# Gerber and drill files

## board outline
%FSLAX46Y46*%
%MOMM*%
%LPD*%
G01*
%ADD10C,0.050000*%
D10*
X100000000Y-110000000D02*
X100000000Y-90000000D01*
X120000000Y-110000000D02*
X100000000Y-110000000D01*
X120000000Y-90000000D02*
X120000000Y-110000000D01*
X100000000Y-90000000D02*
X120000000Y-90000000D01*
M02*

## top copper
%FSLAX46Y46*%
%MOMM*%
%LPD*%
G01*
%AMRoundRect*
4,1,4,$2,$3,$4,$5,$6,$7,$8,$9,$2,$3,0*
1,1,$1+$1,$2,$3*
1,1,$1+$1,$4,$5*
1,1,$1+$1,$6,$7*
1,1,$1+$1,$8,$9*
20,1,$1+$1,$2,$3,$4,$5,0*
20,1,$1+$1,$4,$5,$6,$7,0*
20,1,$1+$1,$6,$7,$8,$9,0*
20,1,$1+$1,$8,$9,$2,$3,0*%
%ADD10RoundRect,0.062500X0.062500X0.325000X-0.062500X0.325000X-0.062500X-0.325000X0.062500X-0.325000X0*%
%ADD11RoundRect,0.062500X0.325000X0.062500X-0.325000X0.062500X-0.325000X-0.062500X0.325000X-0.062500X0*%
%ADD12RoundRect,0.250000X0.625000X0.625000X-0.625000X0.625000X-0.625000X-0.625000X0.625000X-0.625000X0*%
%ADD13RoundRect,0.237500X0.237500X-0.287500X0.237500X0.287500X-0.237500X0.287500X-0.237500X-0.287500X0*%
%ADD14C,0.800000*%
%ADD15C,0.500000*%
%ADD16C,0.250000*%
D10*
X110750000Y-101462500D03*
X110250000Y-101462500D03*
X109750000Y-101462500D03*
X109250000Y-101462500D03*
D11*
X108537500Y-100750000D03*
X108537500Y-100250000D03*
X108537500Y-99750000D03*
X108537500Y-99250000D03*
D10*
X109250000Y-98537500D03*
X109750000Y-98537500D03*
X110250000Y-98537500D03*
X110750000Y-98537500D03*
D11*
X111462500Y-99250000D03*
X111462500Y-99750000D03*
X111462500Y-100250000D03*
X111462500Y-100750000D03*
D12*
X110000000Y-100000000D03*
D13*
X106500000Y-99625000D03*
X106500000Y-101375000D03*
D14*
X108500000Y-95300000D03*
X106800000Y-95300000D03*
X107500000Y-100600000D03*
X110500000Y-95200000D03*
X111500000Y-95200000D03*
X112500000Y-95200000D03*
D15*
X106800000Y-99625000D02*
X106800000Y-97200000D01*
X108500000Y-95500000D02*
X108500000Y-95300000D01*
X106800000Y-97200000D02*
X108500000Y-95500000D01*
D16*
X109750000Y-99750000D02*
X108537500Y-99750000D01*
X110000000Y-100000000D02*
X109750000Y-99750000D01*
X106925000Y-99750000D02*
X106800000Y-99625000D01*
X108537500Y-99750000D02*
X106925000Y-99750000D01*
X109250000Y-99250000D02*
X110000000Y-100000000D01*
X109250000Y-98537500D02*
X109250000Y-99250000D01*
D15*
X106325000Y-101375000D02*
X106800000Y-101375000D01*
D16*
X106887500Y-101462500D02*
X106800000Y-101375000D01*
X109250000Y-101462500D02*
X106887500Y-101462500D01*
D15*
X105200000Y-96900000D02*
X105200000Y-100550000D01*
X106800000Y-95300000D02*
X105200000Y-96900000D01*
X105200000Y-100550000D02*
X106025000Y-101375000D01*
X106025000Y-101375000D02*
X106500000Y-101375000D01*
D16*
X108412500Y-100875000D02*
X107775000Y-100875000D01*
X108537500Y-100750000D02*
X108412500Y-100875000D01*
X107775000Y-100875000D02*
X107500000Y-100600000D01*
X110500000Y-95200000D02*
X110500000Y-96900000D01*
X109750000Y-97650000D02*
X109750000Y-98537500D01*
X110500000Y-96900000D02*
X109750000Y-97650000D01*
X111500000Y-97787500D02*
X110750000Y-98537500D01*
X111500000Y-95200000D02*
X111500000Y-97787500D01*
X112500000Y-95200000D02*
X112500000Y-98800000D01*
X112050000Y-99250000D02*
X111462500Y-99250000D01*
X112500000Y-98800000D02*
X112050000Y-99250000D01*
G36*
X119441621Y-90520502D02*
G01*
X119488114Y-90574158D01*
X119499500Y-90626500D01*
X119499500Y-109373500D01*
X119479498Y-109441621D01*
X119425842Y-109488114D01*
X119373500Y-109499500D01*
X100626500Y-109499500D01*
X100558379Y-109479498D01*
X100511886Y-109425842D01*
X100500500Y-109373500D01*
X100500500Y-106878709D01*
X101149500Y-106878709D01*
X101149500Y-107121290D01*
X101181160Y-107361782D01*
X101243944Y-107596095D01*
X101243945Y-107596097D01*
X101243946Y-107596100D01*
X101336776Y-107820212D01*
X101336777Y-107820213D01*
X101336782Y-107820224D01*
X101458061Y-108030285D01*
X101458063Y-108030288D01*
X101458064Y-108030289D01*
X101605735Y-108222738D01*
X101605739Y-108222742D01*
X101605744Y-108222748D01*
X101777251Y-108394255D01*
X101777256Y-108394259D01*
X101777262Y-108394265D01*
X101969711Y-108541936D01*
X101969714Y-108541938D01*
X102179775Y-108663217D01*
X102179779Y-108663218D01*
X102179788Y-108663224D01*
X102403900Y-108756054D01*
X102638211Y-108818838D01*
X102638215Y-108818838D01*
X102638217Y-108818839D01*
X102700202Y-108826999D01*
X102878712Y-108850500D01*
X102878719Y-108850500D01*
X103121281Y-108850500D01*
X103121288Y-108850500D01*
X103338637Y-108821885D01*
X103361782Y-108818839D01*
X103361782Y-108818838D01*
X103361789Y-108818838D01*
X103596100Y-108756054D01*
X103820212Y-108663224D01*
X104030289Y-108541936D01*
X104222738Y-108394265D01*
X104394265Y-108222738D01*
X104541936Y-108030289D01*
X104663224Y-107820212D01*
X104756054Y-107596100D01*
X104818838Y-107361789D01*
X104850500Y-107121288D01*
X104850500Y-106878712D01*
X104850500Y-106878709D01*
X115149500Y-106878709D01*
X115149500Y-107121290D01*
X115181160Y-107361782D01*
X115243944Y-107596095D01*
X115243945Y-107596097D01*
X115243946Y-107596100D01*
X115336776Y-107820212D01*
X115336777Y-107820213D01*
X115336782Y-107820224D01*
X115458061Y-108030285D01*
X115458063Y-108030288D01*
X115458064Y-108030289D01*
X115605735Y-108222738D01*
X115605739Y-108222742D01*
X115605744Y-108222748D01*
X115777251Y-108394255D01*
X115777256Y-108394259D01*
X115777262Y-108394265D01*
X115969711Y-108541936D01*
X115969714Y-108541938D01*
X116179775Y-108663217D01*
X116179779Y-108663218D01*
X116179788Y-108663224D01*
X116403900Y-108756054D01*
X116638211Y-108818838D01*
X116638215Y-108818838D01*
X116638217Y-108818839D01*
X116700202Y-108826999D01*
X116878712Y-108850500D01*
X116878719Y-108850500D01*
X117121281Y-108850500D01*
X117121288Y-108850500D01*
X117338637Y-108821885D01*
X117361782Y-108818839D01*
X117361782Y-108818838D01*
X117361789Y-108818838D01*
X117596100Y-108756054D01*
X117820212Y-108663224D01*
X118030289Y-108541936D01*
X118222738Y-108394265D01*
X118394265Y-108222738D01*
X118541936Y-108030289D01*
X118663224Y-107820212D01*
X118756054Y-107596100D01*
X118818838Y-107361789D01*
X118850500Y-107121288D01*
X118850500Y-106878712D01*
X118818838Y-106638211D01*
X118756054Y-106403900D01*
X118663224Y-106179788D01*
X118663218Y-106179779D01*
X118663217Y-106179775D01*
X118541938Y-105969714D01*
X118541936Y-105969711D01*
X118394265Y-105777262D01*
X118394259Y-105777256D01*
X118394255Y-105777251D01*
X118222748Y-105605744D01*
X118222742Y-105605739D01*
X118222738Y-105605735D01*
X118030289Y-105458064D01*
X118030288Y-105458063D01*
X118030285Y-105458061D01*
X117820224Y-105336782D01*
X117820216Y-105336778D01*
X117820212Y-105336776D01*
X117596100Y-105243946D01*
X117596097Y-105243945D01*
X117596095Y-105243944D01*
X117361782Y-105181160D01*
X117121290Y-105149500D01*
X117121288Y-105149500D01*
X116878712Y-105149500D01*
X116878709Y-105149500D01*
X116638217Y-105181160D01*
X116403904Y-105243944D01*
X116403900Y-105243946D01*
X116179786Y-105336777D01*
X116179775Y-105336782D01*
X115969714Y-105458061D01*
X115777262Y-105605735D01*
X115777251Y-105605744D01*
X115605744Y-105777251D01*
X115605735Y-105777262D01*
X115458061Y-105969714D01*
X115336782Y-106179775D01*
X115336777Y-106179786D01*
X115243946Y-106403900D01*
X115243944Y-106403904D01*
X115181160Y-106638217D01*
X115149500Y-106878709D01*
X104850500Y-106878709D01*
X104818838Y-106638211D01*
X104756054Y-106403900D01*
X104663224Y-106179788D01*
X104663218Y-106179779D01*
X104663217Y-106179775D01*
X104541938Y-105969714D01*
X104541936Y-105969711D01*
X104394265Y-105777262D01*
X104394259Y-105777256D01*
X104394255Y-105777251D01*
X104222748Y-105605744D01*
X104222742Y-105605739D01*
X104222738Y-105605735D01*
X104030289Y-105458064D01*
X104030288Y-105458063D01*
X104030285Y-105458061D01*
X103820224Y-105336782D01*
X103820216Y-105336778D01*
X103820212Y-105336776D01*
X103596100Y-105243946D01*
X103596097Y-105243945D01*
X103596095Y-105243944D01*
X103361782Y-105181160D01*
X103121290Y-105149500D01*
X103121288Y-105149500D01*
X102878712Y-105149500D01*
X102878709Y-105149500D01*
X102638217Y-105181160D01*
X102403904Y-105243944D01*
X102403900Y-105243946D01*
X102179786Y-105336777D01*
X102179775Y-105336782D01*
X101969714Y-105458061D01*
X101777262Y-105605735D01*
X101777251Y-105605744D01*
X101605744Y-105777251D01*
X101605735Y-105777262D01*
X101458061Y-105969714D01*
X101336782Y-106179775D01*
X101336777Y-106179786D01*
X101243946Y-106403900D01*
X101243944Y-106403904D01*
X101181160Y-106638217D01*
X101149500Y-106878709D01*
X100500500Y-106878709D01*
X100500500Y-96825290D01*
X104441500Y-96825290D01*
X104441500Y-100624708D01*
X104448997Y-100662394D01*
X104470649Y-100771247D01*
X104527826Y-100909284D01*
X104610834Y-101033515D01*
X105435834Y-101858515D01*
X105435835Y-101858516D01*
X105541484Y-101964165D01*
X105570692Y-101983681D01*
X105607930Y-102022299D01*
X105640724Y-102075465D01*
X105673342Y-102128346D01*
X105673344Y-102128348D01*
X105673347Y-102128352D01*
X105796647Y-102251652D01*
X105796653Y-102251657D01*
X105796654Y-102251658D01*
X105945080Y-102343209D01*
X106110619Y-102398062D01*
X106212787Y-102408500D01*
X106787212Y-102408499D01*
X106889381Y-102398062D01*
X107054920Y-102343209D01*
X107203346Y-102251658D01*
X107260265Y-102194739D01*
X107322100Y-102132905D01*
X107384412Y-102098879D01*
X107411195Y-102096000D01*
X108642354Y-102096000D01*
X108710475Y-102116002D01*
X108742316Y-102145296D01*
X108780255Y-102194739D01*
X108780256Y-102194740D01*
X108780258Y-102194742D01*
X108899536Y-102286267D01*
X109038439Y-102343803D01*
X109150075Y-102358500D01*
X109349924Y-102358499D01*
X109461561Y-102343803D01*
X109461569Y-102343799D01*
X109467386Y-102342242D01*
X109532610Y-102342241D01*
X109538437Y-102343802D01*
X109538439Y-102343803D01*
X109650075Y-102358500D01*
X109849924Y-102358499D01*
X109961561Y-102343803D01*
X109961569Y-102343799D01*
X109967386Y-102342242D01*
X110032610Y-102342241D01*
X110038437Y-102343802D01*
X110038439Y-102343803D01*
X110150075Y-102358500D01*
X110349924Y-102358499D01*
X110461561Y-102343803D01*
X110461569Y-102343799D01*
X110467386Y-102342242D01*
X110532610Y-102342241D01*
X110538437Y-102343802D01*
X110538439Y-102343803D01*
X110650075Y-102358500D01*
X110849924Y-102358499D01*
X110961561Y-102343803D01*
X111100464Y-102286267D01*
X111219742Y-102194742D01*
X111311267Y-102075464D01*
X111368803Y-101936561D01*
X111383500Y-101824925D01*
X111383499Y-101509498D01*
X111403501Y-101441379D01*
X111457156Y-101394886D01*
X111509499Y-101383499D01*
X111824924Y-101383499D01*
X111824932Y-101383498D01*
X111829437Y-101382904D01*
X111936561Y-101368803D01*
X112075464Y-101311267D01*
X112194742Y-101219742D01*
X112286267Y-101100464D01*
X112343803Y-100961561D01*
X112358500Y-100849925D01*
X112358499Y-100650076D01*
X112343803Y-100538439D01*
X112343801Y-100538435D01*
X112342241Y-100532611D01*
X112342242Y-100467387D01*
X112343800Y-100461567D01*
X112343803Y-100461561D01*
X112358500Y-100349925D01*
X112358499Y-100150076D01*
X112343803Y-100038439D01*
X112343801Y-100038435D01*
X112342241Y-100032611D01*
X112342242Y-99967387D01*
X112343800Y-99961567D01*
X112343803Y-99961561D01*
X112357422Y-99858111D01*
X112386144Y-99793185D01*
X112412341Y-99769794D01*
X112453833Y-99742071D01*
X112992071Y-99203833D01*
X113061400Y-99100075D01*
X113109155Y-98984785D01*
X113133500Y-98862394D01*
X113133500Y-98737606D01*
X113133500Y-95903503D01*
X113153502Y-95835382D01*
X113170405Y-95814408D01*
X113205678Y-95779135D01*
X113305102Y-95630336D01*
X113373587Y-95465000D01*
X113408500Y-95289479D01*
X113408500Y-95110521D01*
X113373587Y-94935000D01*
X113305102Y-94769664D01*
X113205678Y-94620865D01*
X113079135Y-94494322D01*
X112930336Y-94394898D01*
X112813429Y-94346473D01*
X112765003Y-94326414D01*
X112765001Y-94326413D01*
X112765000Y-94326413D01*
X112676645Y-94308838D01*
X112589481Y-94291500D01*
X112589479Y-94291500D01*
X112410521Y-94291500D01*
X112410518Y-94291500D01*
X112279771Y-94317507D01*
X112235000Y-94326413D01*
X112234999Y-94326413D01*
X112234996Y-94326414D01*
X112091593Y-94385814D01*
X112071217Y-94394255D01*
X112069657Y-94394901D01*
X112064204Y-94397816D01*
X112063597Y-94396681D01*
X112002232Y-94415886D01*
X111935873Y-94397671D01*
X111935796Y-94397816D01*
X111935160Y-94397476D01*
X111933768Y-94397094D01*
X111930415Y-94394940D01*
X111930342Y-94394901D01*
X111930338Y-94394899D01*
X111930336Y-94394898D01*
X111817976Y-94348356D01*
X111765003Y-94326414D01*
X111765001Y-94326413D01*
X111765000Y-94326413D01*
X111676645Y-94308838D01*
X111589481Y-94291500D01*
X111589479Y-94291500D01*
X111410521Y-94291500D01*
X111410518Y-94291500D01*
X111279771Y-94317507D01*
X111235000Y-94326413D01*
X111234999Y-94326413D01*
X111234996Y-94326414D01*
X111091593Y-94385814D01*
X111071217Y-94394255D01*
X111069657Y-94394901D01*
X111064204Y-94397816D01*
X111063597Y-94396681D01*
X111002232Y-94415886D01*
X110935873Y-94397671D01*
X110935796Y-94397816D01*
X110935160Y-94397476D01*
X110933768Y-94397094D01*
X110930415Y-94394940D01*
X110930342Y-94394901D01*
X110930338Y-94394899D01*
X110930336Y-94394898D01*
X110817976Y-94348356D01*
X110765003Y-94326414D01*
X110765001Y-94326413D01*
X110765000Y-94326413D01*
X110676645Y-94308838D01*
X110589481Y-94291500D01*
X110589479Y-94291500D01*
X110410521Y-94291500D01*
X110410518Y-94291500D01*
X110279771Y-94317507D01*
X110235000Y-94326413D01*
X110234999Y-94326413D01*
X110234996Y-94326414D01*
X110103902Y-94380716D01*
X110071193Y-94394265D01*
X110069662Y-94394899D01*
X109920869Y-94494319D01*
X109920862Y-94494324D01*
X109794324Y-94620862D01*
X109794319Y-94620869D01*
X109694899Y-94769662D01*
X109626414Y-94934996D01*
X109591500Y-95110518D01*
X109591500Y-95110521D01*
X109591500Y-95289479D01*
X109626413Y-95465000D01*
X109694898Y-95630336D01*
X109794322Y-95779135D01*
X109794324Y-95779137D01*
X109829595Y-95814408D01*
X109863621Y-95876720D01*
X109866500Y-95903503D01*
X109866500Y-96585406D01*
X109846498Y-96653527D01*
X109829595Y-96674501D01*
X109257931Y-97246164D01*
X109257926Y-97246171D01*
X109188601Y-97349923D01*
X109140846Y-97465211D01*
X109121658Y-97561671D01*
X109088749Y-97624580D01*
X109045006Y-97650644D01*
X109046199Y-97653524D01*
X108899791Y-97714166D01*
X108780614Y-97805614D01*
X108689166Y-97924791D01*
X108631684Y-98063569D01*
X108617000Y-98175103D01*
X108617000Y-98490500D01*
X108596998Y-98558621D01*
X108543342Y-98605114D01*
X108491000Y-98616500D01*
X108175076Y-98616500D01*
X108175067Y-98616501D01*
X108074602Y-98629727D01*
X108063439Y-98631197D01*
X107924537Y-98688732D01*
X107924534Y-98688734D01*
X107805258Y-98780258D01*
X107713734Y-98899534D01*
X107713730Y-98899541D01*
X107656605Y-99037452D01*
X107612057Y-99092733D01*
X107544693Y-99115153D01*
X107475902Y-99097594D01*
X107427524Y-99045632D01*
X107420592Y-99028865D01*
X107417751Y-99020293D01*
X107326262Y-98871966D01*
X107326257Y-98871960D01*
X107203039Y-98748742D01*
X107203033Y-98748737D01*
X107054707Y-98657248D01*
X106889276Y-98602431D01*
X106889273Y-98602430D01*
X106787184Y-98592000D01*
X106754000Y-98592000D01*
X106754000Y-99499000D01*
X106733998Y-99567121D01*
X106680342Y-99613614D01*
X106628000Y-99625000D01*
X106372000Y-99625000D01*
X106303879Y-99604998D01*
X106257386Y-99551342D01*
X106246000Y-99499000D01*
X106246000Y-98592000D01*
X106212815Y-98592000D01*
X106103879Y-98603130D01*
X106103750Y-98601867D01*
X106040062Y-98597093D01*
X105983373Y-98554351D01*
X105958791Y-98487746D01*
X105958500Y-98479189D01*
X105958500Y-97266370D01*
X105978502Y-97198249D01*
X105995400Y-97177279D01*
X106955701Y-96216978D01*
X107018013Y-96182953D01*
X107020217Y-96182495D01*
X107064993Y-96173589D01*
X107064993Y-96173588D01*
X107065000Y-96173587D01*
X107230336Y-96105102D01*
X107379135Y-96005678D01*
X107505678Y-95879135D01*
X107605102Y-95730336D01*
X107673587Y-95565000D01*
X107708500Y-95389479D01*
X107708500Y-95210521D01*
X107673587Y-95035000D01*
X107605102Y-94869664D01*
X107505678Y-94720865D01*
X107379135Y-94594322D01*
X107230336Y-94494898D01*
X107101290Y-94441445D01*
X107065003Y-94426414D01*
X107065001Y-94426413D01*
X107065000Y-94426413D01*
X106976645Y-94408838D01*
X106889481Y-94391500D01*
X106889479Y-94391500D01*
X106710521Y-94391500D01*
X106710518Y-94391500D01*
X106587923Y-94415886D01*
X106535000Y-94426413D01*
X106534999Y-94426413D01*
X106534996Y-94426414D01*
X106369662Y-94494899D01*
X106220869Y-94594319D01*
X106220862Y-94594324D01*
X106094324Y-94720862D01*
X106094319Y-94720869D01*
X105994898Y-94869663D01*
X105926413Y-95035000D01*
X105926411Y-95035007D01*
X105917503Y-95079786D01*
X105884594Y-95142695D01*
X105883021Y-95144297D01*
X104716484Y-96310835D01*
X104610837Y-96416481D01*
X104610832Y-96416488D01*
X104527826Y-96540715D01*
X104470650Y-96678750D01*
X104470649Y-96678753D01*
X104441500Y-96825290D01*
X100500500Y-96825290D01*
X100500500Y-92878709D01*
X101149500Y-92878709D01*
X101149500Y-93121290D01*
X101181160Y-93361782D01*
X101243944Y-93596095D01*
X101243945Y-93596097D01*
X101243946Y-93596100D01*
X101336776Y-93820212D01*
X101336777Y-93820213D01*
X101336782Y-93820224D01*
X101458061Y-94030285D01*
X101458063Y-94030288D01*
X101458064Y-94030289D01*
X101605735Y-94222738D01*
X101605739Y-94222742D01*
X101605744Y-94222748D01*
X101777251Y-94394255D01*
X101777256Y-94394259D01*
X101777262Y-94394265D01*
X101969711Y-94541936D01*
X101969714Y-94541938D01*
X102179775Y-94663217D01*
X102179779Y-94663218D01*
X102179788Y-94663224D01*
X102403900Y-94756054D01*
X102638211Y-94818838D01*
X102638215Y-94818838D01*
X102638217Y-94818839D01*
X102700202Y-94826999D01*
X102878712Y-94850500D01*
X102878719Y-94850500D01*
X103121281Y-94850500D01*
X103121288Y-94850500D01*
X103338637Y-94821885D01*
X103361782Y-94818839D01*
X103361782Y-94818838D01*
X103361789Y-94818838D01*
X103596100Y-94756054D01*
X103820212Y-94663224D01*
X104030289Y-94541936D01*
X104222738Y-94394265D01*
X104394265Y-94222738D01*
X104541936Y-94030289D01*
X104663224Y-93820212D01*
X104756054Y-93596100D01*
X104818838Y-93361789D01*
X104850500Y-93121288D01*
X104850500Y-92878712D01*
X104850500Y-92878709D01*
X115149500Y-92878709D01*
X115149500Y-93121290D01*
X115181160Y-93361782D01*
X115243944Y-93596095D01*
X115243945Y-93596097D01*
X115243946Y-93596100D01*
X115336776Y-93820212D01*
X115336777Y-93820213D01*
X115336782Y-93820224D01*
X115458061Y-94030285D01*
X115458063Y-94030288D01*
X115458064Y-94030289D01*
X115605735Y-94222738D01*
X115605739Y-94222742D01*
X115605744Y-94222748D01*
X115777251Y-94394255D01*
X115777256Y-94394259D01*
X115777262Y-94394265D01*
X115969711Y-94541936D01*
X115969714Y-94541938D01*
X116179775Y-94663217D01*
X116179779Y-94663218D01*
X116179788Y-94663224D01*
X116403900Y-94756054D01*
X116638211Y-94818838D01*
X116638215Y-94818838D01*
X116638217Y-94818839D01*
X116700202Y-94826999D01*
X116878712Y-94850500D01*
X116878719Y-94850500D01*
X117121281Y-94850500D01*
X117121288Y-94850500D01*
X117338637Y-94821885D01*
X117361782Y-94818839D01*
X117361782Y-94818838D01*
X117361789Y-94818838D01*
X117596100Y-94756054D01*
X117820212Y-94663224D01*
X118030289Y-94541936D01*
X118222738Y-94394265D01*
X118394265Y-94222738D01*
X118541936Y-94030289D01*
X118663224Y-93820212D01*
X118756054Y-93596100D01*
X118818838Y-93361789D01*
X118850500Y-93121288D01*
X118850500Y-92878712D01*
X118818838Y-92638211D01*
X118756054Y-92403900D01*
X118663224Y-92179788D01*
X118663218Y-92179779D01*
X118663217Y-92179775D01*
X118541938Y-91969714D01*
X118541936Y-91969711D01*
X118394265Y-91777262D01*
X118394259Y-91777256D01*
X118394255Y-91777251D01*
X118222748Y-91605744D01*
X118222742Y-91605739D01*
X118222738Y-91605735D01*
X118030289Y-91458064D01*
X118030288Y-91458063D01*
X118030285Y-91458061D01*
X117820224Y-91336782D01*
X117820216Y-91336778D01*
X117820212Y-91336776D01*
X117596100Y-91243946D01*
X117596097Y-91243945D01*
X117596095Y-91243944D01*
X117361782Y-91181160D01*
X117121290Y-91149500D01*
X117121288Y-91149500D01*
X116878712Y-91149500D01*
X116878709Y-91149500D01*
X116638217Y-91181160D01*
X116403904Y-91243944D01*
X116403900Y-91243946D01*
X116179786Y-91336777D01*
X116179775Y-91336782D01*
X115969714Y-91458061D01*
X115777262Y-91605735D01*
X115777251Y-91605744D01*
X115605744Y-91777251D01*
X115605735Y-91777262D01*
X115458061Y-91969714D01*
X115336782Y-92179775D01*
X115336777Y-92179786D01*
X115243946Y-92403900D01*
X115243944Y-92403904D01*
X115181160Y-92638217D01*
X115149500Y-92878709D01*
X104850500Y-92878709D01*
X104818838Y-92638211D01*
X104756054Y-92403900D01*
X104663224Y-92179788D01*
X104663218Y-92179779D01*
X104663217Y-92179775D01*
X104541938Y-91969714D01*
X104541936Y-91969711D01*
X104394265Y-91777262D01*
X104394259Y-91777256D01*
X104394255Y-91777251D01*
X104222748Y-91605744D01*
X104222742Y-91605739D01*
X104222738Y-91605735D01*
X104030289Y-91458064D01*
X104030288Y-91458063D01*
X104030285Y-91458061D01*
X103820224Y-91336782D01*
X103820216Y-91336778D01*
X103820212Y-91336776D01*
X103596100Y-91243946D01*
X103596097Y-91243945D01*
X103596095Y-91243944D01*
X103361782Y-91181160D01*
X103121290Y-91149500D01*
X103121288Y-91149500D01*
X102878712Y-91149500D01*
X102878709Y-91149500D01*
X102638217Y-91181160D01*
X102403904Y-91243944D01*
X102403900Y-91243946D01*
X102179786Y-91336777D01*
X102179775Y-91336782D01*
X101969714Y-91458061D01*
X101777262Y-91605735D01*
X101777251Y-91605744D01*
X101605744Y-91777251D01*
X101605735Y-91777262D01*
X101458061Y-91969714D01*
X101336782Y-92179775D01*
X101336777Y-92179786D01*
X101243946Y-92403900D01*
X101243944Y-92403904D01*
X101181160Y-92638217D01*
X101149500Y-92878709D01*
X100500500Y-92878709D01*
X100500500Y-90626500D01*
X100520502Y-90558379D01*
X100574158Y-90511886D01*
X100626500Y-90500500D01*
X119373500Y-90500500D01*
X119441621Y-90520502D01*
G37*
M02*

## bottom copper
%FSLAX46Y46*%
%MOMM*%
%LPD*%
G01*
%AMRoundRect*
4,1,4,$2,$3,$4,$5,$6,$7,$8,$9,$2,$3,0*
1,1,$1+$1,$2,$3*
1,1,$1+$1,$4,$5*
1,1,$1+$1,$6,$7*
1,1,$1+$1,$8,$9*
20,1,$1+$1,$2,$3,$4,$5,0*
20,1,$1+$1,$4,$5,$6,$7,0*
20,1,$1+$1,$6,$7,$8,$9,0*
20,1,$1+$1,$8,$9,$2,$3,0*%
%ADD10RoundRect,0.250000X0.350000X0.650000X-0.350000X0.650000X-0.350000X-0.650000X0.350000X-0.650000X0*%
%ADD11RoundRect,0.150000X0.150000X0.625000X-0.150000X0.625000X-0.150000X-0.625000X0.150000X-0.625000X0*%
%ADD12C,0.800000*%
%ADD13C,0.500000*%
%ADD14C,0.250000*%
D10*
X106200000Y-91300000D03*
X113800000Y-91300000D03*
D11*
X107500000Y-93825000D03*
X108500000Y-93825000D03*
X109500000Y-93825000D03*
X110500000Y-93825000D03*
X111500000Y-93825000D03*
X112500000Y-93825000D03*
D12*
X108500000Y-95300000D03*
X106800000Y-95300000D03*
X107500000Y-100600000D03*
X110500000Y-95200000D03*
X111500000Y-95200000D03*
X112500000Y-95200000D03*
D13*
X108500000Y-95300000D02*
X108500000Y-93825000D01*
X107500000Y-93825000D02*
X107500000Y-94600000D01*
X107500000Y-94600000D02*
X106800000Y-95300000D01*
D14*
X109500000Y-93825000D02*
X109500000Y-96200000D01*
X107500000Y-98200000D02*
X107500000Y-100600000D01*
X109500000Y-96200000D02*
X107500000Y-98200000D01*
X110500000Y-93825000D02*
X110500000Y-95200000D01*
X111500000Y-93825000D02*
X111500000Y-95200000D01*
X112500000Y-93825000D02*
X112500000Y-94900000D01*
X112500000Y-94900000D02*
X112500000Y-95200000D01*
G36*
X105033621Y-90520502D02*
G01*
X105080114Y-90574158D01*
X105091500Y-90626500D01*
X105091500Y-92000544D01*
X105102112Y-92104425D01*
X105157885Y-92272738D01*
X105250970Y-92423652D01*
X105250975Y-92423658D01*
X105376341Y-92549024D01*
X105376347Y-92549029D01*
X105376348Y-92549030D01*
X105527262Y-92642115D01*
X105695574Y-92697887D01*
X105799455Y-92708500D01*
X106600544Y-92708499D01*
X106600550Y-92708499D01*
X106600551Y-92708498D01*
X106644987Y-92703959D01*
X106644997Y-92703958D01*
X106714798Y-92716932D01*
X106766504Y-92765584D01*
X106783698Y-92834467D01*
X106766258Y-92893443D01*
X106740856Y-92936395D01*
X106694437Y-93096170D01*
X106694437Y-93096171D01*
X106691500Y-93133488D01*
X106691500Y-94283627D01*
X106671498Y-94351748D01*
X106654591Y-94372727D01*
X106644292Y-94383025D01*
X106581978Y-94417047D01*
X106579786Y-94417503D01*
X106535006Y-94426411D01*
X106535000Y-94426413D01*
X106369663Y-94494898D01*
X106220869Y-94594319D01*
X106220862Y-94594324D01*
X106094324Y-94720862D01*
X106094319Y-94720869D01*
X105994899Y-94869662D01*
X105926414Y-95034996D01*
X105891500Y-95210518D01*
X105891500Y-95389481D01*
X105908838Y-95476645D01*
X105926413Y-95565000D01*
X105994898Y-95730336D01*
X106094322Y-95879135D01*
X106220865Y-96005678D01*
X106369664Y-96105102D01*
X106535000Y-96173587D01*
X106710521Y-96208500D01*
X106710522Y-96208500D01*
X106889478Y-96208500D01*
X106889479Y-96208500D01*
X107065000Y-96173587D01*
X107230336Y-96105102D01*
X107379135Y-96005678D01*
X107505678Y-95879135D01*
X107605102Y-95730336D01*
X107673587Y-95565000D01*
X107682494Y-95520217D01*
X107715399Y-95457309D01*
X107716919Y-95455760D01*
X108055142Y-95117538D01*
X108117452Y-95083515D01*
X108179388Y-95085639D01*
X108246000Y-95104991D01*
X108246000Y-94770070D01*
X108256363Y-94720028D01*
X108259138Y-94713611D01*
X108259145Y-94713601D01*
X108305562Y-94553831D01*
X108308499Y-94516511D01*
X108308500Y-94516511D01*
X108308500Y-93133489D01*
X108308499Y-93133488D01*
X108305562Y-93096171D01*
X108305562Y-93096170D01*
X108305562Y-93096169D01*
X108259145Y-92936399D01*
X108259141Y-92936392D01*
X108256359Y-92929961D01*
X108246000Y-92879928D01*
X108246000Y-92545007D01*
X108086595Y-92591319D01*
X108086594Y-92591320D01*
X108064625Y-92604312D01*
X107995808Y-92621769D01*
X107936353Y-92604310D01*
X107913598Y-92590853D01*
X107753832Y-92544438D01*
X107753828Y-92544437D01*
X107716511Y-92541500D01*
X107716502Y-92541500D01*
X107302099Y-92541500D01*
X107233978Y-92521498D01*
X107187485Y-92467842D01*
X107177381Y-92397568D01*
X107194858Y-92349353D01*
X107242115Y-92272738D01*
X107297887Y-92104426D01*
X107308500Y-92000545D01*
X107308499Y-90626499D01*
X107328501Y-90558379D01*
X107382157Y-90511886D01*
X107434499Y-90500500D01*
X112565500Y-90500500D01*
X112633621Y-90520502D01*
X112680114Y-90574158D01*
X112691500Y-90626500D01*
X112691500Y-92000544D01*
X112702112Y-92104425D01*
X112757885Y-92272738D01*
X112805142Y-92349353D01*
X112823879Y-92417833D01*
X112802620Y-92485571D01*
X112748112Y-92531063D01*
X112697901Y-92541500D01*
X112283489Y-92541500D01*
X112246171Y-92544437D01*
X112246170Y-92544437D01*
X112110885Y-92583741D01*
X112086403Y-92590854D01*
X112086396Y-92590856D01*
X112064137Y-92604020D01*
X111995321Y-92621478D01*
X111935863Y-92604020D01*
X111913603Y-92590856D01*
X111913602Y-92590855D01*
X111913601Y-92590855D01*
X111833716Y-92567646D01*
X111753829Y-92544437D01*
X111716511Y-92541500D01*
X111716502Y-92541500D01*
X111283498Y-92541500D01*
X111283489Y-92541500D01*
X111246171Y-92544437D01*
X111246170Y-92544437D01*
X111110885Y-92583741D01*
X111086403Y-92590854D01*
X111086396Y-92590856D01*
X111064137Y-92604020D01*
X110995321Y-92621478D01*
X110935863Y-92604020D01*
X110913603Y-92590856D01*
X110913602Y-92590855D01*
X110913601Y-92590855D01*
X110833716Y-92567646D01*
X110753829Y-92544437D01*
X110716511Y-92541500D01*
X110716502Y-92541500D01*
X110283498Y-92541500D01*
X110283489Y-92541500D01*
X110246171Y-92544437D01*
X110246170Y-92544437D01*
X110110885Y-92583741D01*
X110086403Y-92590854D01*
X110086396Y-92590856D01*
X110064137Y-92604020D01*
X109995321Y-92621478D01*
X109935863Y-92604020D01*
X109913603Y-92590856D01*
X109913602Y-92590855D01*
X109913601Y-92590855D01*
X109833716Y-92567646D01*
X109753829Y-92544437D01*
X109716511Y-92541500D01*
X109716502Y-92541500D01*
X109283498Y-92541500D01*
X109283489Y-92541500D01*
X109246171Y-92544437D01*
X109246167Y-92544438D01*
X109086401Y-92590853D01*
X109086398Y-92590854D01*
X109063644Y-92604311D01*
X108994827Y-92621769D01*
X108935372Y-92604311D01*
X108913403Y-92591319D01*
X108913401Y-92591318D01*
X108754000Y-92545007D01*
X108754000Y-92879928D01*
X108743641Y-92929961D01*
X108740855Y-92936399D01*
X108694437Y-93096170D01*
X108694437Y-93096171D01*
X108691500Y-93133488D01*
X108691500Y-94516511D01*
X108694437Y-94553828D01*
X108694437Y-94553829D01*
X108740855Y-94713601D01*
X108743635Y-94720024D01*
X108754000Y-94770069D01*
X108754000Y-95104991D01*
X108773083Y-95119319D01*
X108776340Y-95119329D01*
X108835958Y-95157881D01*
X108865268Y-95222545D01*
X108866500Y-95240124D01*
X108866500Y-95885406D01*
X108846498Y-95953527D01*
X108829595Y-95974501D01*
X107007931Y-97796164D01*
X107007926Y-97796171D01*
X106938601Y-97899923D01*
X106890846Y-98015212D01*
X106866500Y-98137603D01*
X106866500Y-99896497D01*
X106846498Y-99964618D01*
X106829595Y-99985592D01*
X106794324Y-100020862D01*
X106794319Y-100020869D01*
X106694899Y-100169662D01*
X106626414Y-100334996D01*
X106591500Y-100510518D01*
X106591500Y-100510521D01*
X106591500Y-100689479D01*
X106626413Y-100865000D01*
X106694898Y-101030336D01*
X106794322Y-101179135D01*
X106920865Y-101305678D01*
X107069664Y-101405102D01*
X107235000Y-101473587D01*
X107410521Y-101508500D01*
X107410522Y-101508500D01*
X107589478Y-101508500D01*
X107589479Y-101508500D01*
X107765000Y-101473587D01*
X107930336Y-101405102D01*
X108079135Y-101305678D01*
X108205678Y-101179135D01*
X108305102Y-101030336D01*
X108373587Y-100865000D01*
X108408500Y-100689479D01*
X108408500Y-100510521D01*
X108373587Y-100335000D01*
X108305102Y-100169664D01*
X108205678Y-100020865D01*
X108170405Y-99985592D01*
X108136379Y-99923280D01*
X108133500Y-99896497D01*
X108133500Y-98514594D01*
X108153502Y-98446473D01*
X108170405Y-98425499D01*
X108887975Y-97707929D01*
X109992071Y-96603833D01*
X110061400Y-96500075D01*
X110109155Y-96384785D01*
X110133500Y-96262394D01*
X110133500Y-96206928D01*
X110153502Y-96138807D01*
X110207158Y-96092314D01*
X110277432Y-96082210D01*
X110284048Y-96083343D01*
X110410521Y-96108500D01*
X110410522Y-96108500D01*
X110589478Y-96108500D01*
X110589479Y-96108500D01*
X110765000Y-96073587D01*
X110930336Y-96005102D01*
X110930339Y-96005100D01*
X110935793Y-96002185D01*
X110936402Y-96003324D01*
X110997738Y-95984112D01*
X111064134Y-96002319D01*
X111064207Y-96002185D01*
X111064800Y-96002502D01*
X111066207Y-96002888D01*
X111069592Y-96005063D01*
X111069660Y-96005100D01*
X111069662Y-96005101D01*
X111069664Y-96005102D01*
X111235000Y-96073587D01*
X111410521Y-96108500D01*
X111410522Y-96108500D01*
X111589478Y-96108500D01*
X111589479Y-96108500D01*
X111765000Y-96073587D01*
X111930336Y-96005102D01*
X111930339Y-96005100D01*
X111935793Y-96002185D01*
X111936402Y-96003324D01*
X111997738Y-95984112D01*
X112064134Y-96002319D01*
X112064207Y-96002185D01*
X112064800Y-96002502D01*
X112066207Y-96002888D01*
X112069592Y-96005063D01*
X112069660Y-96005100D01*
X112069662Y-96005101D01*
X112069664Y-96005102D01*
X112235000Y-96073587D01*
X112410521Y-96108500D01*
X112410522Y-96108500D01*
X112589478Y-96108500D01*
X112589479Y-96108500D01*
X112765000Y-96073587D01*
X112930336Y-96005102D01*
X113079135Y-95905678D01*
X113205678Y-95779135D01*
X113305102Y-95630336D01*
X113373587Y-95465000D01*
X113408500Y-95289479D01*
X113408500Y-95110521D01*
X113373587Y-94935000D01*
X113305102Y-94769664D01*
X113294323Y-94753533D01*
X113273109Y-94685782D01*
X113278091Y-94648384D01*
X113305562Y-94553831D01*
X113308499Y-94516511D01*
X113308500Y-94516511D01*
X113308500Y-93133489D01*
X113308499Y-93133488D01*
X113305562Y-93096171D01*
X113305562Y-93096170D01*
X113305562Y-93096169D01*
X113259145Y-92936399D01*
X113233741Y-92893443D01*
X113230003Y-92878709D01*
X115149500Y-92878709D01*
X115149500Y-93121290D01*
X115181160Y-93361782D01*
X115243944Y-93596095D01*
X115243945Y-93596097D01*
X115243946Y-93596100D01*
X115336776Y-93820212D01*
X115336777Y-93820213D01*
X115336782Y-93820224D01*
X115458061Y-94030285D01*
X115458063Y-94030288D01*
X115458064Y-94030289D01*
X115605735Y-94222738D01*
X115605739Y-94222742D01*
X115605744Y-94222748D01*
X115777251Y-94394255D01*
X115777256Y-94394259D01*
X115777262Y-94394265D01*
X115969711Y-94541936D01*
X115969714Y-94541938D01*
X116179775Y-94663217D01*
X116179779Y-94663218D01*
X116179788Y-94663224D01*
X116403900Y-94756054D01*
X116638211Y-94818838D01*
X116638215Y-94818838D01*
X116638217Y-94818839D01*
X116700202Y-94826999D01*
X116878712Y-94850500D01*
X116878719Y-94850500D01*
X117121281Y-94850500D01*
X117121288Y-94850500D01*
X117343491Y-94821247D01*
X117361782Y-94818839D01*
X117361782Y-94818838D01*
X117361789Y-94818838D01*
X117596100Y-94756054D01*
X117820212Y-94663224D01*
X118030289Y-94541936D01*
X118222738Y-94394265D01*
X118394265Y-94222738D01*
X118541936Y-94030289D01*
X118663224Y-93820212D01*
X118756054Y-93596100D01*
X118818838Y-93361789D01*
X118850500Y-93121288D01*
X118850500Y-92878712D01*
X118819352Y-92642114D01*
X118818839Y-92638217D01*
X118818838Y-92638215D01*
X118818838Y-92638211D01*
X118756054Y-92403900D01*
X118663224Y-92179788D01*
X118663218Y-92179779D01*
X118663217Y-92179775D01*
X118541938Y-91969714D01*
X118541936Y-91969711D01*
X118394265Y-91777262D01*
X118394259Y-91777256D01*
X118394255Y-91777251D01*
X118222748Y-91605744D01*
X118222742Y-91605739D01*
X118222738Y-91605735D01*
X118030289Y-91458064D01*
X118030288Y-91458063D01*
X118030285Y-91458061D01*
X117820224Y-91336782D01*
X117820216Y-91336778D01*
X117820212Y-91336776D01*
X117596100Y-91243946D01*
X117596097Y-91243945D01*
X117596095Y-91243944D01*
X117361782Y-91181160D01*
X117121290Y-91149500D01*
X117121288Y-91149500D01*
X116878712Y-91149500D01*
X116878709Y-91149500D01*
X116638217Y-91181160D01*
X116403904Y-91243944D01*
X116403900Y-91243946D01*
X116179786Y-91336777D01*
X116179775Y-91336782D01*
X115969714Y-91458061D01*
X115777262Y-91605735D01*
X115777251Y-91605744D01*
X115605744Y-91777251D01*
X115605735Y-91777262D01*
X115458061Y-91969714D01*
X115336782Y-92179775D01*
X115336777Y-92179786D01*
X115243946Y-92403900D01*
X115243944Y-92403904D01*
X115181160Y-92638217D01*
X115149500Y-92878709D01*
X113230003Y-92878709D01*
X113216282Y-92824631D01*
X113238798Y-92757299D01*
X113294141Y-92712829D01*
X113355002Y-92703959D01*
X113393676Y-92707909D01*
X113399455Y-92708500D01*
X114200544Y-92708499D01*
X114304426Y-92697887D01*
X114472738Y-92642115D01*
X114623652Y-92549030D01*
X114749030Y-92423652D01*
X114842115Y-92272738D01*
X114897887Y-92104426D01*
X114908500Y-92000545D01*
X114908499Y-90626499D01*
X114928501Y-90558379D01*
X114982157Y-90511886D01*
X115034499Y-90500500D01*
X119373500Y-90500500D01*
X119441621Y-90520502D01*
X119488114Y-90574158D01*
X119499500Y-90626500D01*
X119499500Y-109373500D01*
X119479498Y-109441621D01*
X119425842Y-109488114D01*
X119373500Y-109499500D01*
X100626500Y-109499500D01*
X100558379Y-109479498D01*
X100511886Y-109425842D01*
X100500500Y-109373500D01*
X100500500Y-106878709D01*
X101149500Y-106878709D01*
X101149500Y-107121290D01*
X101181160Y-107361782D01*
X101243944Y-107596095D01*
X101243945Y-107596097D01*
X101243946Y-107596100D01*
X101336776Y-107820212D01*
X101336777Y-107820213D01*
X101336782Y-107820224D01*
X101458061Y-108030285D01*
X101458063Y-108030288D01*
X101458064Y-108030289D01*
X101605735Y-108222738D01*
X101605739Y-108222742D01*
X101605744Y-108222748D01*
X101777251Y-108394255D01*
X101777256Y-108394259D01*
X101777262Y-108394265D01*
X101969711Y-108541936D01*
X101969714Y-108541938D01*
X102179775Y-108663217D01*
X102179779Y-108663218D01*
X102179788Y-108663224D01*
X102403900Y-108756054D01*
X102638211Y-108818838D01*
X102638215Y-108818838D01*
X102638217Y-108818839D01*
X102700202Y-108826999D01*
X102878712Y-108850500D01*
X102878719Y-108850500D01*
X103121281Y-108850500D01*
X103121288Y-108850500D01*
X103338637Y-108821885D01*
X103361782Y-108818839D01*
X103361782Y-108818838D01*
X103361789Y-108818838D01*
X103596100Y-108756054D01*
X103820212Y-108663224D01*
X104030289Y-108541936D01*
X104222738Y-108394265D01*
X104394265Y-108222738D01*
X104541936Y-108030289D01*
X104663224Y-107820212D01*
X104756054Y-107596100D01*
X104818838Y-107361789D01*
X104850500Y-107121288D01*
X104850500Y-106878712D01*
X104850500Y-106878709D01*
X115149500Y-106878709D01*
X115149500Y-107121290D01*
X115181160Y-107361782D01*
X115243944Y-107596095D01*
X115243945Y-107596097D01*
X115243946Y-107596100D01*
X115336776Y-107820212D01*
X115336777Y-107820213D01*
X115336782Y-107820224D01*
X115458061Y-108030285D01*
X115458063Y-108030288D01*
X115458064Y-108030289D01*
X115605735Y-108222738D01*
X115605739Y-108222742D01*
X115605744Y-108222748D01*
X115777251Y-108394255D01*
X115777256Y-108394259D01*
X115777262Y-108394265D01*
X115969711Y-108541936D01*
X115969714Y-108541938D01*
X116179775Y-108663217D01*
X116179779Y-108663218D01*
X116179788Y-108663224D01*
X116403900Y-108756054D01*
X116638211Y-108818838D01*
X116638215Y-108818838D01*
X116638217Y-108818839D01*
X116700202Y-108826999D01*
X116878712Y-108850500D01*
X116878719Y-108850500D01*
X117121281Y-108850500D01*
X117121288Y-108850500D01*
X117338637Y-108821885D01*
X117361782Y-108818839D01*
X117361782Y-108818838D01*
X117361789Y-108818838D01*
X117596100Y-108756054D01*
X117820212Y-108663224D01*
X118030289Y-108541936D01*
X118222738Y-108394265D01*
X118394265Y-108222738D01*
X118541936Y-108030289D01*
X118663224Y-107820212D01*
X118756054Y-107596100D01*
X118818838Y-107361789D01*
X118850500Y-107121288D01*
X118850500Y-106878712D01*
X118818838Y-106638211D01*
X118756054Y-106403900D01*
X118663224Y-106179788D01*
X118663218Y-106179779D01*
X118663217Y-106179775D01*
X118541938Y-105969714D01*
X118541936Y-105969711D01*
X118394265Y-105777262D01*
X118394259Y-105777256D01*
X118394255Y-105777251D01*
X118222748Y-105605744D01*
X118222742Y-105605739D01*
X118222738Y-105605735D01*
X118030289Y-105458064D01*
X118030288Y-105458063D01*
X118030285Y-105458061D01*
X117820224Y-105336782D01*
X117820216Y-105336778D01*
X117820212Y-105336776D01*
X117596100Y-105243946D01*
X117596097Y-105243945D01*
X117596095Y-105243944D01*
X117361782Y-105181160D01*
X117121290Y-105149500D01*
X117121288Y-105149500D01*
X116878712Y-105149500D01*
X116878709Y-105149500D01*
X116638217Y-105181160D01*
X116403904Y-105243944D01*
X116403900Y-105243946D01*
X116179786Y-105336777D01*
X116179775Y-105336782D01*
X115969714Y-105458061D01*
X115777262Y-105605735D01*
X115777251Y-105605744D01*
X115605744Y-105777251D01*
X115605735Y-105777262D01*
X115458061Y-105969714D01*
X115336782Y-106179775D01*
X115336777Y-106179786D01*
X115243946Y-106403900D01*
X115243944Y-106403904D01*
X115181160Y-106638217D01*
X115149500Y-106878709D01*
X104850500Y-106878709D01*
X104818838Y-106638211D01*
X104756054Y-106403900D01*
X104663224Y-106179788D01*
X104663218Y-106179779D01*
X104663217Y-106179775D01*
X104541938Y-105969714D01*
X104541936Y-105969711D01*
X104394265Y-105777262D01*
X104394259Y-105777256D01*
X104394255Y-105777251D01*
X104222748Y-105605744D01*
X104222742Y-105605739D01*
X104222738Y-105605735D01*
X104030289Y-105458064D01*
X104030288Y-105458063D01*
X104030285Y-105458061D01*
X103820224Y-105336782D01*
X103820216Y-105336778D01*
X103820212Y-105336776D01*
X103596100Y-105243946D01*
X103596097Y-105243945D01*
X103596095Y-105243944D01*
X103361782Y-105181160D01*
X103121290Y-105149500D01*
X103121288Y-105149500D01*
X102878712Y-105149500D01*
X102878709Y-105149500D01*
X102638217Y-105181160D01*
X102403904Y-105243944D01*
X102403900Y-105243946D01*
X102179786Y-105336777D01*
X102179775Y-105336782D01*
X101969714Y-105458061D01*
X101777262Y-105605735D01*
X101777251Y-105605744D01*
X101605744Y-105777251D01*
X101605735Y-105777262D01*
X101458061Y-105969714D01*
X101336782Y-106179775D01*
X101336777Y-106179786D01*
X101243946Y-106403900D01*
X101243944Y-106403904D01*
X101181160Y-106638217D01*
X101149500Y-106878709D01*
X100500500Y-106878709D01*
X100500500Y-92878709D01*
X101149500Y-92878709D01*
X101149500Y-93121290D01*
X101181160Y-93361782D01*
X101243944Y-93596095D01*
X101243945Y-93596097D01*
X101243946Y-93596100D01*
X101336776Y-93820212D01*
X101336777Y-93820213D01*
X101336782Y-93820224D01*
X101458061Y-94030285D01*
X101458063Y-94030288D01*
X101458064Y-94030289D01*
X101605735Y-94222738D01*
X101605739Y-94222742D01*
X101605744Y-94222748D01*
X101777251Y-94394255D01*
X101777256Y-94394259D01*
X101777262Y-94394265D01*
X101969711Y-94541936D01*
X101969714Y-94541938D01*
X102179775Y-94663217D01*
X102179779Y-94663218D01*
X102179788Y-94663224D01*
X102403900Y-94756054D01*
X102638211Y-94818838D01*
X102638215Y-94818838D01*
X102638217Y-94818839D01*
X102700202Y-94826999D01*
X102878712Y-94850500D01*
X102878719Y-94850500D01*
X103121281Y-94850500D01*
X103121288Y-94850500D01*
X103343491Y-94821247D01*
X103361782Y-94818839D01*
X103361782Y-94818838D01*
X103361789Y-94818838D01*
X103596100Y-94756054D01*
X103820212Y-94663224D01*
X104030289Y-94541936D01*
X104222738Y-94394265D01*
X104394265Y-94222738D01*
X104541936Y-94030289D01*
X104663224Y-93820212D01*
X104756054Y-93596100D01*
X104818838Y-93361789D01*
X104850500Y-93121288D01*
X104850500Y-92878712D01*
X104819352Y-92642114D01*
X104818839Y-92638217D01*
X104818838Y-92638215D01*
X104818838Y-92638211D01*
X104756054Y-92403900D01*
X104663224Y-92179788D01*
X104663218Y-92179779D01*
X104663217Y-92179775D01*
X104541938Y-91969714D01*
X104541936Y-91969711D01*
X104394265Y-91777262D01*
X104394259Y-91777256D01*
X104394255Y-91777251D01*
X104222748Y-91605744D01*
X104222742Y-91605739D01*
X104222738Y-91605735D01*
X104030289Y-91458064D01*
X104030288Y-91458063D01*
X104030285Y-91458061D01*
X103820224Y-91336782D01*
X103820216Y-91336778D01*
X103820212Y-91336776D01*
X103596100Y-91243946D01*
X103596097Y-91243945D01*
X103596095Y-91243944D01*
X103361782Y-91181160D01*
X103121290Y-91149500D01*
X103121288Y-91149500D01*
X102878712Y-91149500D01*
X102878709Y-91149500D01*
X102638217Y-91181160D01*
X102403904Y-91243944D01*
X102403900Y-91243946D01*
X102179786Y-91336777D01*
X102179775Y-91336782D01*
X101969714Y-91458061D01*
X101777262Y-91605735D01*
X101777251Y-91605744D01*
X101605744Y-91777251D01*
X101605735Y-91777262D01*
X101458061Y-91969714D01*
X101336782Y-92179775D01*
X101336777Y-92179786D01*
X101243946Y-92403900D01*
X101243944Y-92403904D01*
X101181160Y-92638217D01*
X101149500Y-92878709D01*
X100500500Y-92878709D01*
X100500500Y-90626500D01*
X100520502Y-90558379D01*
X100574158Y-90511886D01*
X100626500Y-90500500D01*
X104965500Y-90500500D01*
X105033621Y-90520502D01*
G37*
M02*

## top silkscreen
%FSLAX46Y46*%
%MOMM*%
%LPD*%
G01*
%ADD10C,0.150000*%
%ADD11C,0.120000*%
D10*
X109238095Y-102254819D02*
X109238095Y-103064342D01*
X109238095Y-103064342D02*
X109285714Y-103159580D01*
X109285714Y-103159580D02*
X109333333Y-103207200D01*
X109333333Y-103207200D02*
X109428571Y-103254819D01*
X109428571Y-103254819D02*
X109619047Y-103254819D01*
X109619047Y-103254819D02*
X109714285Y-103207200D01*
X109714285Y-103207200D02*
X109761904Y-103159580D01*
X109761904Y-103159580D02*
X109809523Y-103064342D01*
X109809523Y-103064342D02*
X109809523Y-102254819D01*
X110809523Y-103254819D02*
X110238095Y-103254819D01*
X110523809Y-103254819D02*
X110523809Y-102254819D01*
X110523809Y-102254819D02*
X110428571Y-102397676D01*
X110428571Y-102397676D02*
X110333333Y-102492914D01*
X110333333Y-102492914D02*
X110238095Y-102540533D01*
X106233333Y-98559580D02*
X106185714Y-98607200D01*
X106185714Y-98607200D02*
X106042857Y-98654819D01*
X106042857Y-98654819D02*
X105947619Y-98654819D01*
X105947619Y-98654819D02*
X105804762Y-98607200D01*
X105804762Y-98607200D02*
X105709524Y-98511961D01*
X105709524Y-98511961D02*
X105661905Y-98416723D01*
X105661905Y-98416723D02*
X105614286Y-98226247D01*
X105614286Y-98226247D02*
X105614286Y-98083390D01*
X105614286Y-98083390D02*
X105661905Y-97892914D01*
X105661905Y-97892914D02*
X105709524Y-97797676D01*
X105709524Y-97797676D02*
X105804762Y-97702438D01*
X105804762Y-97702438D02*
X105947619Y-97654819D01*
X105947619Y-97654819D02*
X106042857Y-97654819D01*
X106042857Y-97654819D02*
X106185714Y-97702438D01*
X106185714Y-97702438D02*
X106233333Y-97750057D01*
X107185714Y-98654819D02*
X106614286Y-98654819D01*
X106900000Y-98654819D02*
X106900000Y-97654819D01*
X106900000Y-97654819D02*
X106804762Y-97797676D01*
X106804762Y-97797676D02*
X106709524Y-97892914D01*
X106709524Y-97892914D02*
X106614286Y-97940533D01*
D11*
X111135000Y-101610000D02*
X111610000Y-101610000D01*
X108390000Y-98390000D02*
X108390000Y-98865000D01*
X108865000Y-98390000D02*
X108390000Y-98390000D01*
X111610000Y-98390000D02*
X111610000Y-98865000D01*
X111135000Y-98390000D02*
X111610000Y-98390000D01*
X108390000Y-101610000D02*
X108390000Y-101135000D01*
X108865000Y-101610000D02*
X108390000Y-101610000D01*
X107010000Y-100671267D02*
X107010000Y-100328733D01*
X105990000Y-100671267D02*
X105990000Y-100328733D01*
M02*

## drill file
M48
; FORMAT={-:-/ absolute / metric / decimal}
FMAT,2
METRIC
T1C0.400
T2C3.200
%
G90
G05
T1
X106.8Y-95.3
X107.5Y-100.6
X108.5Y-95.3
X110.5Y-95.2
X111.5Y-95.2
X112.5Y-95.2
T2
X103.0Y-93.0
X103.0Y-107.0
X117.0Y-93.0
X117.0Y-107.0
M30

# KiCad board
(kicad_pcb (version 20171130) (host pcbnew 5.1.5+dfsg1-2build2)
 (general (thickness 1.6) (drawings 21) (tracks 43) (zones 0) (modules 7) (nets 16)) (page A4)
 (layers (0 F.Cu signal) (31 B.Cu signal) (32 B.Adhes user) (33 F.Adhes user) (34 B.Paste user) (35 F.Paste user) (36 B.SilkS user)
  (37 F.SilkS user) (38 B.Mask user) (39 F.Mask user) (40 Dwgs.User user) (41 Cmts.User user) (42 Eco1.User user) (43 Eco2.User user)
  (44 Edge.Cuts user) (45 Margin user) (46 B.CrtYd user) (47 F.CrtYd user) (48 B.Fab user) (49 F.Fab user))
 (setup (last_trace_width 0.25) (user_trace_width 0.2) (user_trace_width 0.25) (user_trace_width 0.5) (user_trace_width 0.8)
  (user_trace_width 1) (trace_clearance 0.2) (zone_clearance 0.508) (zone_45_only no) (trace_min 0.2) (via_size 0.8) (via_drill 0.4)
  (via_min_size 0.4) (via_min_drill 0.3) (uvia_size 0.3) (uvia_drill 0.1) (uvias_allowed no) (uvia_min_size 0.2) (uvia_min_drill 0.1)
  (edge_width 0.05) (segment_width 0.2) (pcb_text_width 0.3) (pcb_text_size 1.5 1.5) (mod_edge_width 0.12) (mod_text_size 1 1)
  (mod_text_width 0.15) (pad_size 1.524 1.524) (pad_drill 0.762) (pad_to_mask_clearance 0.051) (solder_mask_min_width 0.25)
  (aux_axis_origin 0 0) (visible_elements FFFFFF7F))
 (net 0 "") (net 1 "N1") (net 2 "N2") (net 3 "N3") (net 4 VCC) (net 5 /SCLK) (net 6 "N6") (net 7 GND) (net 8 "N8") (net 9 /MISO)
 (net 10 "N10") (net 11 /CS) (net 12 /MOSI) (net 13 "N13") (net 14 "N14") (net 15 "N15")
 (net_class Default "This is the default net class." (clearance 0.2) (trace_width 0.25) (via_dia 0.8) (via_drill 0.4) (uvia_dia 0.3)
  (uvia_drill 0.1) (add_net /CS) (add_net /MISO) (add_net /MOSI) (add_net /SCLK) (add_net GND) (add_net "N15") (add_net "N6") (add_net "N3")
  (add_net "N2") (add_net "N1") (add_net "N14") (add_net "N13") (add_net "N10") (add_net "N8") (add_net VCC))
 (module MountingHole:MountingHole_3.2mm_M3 (layer F.Cu) (at 103 107)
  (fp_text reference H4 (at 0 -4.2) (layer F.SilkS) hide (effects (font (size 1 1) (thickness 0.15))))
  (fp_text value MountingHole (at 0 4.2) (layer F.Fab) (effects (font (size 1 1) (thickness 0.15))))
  (pad 1 np_thru_hole circle (at 0 0) (size 3.2 3.2) (drill 3.2) (layers *.Cu *.Mask)))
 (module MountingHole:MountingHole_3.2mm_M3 (layer F.Cu) (at 117 93)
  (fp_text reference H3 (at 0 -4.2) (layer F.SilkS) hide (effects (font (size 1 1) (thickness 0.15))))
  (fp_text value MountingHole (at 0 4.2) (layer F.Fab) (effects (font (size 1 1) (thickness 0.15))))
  (pad 1 np_thru_hole circle (at 0 0) (size 3.2 3.2) (drill 3.2) (layers *.Cu *.Mask)))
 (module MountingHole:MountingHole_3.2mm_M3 (layer F.Cu) (at 103 93)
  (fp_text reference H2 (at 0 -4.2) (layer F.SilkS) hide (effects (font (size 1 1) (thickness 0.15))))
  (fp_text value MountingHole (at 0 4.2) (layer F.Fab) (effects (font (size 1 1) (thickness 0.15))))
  (pad 1 np_thru_hole circle (at 0 0) (size 3.2 3.2) (drill 3.2) (layers *.Cu *.Mask)))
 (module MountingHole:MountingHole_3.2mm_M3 (layer F.Cu) (at 117 107)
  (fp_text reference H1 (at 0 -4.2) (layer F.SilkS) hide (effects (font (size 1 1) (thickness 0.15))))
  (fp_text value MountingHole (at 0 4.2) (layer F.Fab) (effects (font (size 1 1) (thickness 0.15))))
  (pad 1 np_thru_hole circle (at 0 0) (size 3.2 3.2) (drill 3.2) (layers *.Cu *.Mask)))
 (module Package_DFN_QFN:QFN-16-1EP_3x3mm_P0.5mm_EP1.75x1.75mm (layer F.Cu) (at 110 100 180)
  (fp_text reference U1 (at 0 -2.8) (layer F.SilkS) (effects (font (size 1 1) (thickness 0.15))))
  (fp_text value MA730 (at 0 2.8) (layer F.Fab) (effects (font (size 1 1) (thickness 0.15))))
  (fp_line (start -1.135 -1.61) (end -1.61 -1.61) (layer F.SilkS) (width 0.12))
  (fp_line (start 1.61 1.61) (end 1.61 1.135) (layer F.SilkS) (width 0.12))
  (fp_line (start 1.135 1.61) (end 1.61 1.61) (layer F.SilkS) (width 0.12))
  (fp_line (start -1.61 1.61) (end -1.61 1.135) (layer F.SilkS) (width 0.12))
  (fp_line (start -1.135 1.61) (end -1.61 1.61) (layer F.SilkS) (width 0.12))
  (fp_line (start 1.61 -1.61) (end 1.61 -1.135) (layer F.SilkS) (width 0.12))
  (fp_line (start 1.135 -1.61) (end 1.61 -1.61) (layer F.SilkS) (width 0.12))
  (pad 16 smd roundrect (at -0.75 -1.4625 180) (size 0.25 0.775) (layers F.Cu F.Paste F.Mask) (roundrect_rratio 0.25) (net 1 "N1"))
  (pad 15 smd roundrect (at -0.25 -1.4625 180) (size 0.25 0.775) (layers F.Cu F.Paste F.Mask) (roundrect_rratio 0.25) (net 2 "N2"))
  (pad 14 smd roundrect (at 0.25 -1.4625 180) (size 0.25 0.775) (layers F.Cu F.Paste F.Mask) (roundrect_rratio 0.25) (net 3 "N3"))
  (pad 13 smd roundrect (at 0.75 -1.4625 180) (size 0.25 0.775) (layers F.Cu F.Paste F.Mask) (roundrect_rratio 0.25) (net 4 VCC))
  (pad 12 smd roundrect (at 1.4625 -0.75 180) (size 0.775 0.25) (layers F.Cu F.Paste F.Mask) (roundrect_rratio 0.25) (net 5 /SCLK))
  (pad 11 smd roundrect (at 1.4625 -0.25 180) (size 0.775 0.25) (layers F.Cu F.Paste F.Mask) (roundrect_rratio 0.25) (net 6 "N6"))
  (pad 10 smd roundrect (at 1.4625 0.25 180) (size 0.775 0.25) (layers F.Cu F.Paste F.Mask) (roundrect_rratio 0.25) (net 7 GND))
  (pad 9 smd roundrect (at 1.4625 0.75 180) (size 0.775 0.25) (layers F.Cu F.Paste F.Mask) (roundrect_rratio 0.25) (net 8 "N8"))
  (pad 8 smd roundrect (at 0.75 1.4625 180) (size 0.25 0.775) (layers F.Cu F.Paste F.Mask) (roundrect_rratio 0.25) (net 7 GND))
  (pad 7 smd roundrect (at 0.25 1.4625 180) (size 0.25 0.775) (layers F.Cu F.Paste F.Mask) (roundrect_rratio 0.25) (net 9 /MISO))
  (pad 6 smd roundrect (at -0.25 1.4625 180) (size 0.25 0.775) (layers F.Cu F.Paste F.Mask) (roundrect_rratio 0.25) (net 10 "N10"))
  (pad 5 smd roundrect (at -0.75 1.4625 180) (size 0.25 0.775) (layers F.Cu F.Paste F.Mask) (roundrect_rratio 0.25) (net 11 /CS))
  (pad 4 smd roundrect (at -1.4625 0.75 180) (size 0.775 0.25) (layers F.Cu F.Paste F.Mask) (roundrect_rratio 0.25) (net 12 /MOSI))
  (pad 3 smd roundrect (at -1.4625 0.25 180) (size 0.775 0.25) (layers F.Cu F.Paste F.Mask) (roundrect_rratio 0.25) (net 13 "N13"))
  (pad 2 smd roundrect (at -1.4625 -0.25 180) (size 0.775 0.25) (layers F.Cu F.Paste F.Mask) (roundrect_rratio 0.25) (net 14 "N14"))
  (pad 1 smd roundrect (at -1.4625 -0.75 180) (size 0.775 0.25) (layers F.Cu F.Paste F.Mask) (roundrect_rratio 0.25) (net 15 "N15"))
  (pad "" smd roundrect (at 0.44 0.44 180) (size 0.71 0.71) (layers F.Paste) (roundrect_rratio 0.25))
  (pad "" smd roundrect (at 0.44 -0.44 180) (size 0.71 0.71) (layers F.Paste) (roundrect_rratio 0.25))
  (pad "" smd roundrect (at -0.44 0.44 180) (size 0.71 0.71) (layers F.Paste) (roundrect_rratio 0.25))
  (pad "" smd roundrect (at -0.44 -0.44 180) (size 0.71 0.71) (layers F.Paste) (roundrect_rratio 0.25))
  (pad 17 smd roundrect (at 0 0 180) (size 1.75 1.75) (layers F.Cu F.Mask) (roundrect_rratio 0.142857) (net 7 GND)))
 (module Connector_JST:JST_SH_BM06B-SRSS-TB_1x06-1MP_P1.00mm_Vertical (layer B.Cu) (at 110 92.5 180)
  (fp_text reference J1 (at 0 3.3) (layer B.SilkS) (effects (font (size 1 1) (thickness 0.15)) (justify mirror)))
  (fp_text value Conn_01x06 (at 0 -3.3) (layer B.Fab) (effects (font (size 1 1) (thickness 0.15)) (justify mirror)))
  (pad MP smd roundrect (at 3.8 1.2 180) (size 1.2 1.8) (layers B.Cu B.Paste B.Mask) (roundrect_rratio 0.208333))
  (pad MP smd roundrect (at -3.8 1.2 180) (size 1.2 1.8) (layers B.Cu B.Paste B.Mask) (roundrect_rratio 0.208333))
  (pad 6 smd roundrect (at 2.5 -1.325 180) (size 0.6 1.55) (layers B.Cu B.Paste B.Mask) (roundrect_rratio 0.25) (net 4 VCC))
  (pad 5 smd roundrect (at 1.5 -1.325 180) (size 0.6 1.55) (layers B.Cu B.Paste B.Mask) (roundrect_rratio 0.25) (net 7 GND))
  (pad 4 smd roundrect (at 0.5 -1.325 180) (size 0.6 1.55) (layers B.Cu B.Paste B.Mask) (roundrect_rratio 0.25) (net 5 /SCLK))
  (pad 3 smd roundrect (at -0.5 -1.325 180) (size 0.6 1.55) (layers B.Cu B.Paste B.Mask) (roundrect_rratio 0.25) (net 9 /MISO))
  (pad 2 smd roundrect (at -1.5 -1.325 180) (size 0.6 1.55) (layers B.Cu B.Paste B.Mask) (roundrect_rratio 0.25) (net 11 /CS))
  (pad 1 smd roundrect (at -2.5 -1.325 180) (size 0.6 1.55) (layers B.Cu B.Paste B.Mask) (roundrect_rratio 0.25) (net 12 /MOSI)))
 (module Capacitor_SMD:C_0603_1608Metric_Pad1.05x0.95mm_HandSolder (layer F.Cu) (at 106.5 100.5 90)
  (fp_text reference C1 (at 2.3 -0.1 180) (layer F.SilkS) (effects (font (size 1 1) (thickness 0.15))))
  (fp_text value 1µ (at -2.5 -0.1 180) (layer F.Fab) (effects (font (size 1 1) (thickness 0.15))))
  (fp_line (start -0.171267 0.51) (end 0.171267 0.51) (layer F.SilkS) (width 0.12))
  (fp_line (start -0.171267 -0.51) (end 0.171267 -0.51) (layer F.SilkS) (width 0.12))
  (pad 2 smd roundrect (at 0.875 0 90) (size 1.05 0.95) (layers F.Cu F.Paste F.Mask) (roundrect_rratio 0.25) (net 7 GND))
  (pad 1 smd roundrect (at -0.875 0 90) (size 1.05 0.95) (layers F.Cu F.Paste F.Mask) (roundrect_rratio 0.25) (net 4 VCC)))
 (gr_line (start 100 110) (end 100 90) (layer Edge.Cuts) (width 0.05))
 (gr_line (start 120 110) (end 100 110) (layer Edge.Cuts) (width 0.05))
 (gr_line (start 120 90) (end 120 110) (layer Edge.Cuts) (width 0.05))
 (gr_line (start 100 90) (end 120 90) (layer Edge.Cuts) (width 0.05))
 (segment (start 106.8 99.625) (end 106.8 97.2) (width 0.5) (layer F.Cu) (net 7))
 (via (at 108.5 95.3) (size 0.8) (drill 0.4) (layers F.Cu B.Cu) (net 7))
 (segment (start 108.5 95.5) (end 108.5 95.3) (width 0.5) (layer F.Cu) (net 7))
 (segment (start 106.8 97.2) (end 108.5 95.5) (width 0.5) (layer F.Cu) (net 7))
 (segment (start 108.5 95.3) (end 108.5 93.825) (width 0.5) (layer B.Cu) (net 7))
 (segment (start 109.75 99.75) (end 108.5375 99.75) (width 0.25) (layer F.Cu) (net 7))
 (segment (start 110 100) (end 109.75 99.75) (width 0.25) (layer F.Cu) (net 7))
 (segment (start 106.925 99.75) (end 106.8 99.625) (width 0.25) (layer F.Cu) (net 7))
 (segment (start 108.5375 99.75) (end 106.925 99.75) (width 0.25) (layer F.Cu) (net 7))
 (segment (start 109.25 99.25) (end 110 100) (width 0.25) (layer F.Cu) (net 7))
 (segment (start 109.25 98.5375) (end 109.25 99.25) (width 0.25) (layer F.Cu) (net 7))
 (segment (start 106.325 101.375) (end 106.8 101.375) (width 0.5) (layer F.Cu) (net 4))
 (segment (start 106.8875 101.4625) (end 106.8 101.375) (width 0.25) (layer F.Cu) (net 4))
 (segment (start 109.25 101.4625) (end 106.8875 101.4625) (width 0.25) (layer F.Cu) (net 4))
 (segment (start 105.2 96.9) (end 105.2 100.55) (width 0.5) (layer F.Cu) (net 4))
 (segment (start 106.8 95.3) (end 105.2 96.9) (width 0.5) (layer F.Cu) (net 4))
 (via (at 106.8 95.3) (size 0.8) (drill 0.4) (layers F.Cu B.Cu) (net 4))
 (segment (start 105.2 100.55) (end 106.025 101.375) (width 0.5) (layer F.Cu) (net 4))
 (segment (start 107.5 93.825) (end 107.5 94.6) (width 0.5) (layer B.Cu) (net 4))
 (segment (start 107.5 94.6) (end 106.8 95.3) (width 0.5) (layer B.Cu) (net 4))
 (segment (start 106.025 101.375) (end 106.5 101.375) (width 0.5) (layer F.Cu) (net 4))
 (segment (start 108.4125 100.875) (end 107.775 100.875) (width 0.25) (layer F.Cu) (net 5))
 (segment (start 108.5375 100.75) (end 108.4125 100.875) (width 0.25) (layer F.Cu) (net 5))
 (segment (start 107.775 100.875) (end 107.5 100.6) (width 0.25) (layer F.Cu) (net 5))
 (via (at 107.5 100.6) (size 0.8) (drill 0.4) (layers F.Cu B.Cu) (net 5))
 (segment (start 109.5 93.825) (end 109.5 96.2) (width 0.25) (layer B.Cu) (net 5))
 (segment (start 107.5 98.2) (end 107.5 100.6) (width 0.25) (layer B.Cu) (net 5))
 (segment (start 109.5 96.2) (end 107.5 98.2) (width 0.25) (layer B.Cu) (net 5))
 (via (at 110.5 95.2) (size 0.8) (drill 0.4) (layers F.Cu B.Cu) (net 9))
 (segment (start 110.5 93.825) (end 110.5 95.2) (width 0.25) (layer B.Cu) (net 9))
 (segment (start 110.5 95.2) (end 110.5 96.9) (width 0.25) (layer F.Cu) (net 9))
 (segment (start 109.75 97.65) (end 109.75 98.5375) (width 0.25) (layer F.Cu) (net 9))
 (segment (start 110.5 96.9) (end 109.75 97.65) (width 0.25) (layer F.Cu) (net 9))
 (via (at 111.5 95.2) (size 0.8) (drill 0.4) (layers F.Cu B.Cu) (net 11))
 (segment (start 111.5 93.825) (end 111.5 95.2) (width 0.25) (layer B.Cu) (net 11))
 (segment (start 111.5 97.7875) (end 110.75 98.5375) (width 0.25) (layer F.Cu) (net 11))
 (segment (start 111.5 95.2) (end 111.5 97.7875) (width 0.25) (layer F.Cu) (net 11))
 (segment (start 112.5 93.825) (end 112.5 94.9) (width 0.25) (layer B.Cu) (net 12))
 (via (at 112.5 95.2) (size 0.8) (drill 0.4) (layers F.Cu B.Cu) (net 12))
 (segment (start 112.5 94.9) (end 112.5 95.2) (width 0.25) (layer B.Cu) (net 12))
 (segment (start 112.5 95.2) (end 112.5 98.8) (width 0.25) (layer F.Cu) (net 12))
 (segment (start 112.05 99.25) (end 111.4625 99.25) (width 0.25) (layer F.Cu) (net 12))
 (segment (start 112.5 98.8) (end 112.05 99.25) (width 0.25) (layer F.Cu) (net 12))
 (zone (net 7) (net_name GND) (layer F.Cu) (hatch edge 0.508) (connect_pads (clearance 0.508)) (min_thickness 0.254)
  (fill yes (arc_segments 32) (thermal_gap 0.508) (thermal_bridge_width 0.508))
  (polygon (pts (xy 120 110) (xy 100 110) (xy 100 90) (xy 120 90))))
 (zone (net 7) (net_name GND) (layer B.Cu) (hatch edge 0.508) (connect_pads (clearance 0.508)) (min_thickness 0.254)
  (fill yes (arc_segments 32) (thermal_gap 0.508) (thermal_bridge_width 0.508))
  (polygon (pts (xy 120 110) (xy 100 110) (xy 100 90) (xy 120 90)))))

